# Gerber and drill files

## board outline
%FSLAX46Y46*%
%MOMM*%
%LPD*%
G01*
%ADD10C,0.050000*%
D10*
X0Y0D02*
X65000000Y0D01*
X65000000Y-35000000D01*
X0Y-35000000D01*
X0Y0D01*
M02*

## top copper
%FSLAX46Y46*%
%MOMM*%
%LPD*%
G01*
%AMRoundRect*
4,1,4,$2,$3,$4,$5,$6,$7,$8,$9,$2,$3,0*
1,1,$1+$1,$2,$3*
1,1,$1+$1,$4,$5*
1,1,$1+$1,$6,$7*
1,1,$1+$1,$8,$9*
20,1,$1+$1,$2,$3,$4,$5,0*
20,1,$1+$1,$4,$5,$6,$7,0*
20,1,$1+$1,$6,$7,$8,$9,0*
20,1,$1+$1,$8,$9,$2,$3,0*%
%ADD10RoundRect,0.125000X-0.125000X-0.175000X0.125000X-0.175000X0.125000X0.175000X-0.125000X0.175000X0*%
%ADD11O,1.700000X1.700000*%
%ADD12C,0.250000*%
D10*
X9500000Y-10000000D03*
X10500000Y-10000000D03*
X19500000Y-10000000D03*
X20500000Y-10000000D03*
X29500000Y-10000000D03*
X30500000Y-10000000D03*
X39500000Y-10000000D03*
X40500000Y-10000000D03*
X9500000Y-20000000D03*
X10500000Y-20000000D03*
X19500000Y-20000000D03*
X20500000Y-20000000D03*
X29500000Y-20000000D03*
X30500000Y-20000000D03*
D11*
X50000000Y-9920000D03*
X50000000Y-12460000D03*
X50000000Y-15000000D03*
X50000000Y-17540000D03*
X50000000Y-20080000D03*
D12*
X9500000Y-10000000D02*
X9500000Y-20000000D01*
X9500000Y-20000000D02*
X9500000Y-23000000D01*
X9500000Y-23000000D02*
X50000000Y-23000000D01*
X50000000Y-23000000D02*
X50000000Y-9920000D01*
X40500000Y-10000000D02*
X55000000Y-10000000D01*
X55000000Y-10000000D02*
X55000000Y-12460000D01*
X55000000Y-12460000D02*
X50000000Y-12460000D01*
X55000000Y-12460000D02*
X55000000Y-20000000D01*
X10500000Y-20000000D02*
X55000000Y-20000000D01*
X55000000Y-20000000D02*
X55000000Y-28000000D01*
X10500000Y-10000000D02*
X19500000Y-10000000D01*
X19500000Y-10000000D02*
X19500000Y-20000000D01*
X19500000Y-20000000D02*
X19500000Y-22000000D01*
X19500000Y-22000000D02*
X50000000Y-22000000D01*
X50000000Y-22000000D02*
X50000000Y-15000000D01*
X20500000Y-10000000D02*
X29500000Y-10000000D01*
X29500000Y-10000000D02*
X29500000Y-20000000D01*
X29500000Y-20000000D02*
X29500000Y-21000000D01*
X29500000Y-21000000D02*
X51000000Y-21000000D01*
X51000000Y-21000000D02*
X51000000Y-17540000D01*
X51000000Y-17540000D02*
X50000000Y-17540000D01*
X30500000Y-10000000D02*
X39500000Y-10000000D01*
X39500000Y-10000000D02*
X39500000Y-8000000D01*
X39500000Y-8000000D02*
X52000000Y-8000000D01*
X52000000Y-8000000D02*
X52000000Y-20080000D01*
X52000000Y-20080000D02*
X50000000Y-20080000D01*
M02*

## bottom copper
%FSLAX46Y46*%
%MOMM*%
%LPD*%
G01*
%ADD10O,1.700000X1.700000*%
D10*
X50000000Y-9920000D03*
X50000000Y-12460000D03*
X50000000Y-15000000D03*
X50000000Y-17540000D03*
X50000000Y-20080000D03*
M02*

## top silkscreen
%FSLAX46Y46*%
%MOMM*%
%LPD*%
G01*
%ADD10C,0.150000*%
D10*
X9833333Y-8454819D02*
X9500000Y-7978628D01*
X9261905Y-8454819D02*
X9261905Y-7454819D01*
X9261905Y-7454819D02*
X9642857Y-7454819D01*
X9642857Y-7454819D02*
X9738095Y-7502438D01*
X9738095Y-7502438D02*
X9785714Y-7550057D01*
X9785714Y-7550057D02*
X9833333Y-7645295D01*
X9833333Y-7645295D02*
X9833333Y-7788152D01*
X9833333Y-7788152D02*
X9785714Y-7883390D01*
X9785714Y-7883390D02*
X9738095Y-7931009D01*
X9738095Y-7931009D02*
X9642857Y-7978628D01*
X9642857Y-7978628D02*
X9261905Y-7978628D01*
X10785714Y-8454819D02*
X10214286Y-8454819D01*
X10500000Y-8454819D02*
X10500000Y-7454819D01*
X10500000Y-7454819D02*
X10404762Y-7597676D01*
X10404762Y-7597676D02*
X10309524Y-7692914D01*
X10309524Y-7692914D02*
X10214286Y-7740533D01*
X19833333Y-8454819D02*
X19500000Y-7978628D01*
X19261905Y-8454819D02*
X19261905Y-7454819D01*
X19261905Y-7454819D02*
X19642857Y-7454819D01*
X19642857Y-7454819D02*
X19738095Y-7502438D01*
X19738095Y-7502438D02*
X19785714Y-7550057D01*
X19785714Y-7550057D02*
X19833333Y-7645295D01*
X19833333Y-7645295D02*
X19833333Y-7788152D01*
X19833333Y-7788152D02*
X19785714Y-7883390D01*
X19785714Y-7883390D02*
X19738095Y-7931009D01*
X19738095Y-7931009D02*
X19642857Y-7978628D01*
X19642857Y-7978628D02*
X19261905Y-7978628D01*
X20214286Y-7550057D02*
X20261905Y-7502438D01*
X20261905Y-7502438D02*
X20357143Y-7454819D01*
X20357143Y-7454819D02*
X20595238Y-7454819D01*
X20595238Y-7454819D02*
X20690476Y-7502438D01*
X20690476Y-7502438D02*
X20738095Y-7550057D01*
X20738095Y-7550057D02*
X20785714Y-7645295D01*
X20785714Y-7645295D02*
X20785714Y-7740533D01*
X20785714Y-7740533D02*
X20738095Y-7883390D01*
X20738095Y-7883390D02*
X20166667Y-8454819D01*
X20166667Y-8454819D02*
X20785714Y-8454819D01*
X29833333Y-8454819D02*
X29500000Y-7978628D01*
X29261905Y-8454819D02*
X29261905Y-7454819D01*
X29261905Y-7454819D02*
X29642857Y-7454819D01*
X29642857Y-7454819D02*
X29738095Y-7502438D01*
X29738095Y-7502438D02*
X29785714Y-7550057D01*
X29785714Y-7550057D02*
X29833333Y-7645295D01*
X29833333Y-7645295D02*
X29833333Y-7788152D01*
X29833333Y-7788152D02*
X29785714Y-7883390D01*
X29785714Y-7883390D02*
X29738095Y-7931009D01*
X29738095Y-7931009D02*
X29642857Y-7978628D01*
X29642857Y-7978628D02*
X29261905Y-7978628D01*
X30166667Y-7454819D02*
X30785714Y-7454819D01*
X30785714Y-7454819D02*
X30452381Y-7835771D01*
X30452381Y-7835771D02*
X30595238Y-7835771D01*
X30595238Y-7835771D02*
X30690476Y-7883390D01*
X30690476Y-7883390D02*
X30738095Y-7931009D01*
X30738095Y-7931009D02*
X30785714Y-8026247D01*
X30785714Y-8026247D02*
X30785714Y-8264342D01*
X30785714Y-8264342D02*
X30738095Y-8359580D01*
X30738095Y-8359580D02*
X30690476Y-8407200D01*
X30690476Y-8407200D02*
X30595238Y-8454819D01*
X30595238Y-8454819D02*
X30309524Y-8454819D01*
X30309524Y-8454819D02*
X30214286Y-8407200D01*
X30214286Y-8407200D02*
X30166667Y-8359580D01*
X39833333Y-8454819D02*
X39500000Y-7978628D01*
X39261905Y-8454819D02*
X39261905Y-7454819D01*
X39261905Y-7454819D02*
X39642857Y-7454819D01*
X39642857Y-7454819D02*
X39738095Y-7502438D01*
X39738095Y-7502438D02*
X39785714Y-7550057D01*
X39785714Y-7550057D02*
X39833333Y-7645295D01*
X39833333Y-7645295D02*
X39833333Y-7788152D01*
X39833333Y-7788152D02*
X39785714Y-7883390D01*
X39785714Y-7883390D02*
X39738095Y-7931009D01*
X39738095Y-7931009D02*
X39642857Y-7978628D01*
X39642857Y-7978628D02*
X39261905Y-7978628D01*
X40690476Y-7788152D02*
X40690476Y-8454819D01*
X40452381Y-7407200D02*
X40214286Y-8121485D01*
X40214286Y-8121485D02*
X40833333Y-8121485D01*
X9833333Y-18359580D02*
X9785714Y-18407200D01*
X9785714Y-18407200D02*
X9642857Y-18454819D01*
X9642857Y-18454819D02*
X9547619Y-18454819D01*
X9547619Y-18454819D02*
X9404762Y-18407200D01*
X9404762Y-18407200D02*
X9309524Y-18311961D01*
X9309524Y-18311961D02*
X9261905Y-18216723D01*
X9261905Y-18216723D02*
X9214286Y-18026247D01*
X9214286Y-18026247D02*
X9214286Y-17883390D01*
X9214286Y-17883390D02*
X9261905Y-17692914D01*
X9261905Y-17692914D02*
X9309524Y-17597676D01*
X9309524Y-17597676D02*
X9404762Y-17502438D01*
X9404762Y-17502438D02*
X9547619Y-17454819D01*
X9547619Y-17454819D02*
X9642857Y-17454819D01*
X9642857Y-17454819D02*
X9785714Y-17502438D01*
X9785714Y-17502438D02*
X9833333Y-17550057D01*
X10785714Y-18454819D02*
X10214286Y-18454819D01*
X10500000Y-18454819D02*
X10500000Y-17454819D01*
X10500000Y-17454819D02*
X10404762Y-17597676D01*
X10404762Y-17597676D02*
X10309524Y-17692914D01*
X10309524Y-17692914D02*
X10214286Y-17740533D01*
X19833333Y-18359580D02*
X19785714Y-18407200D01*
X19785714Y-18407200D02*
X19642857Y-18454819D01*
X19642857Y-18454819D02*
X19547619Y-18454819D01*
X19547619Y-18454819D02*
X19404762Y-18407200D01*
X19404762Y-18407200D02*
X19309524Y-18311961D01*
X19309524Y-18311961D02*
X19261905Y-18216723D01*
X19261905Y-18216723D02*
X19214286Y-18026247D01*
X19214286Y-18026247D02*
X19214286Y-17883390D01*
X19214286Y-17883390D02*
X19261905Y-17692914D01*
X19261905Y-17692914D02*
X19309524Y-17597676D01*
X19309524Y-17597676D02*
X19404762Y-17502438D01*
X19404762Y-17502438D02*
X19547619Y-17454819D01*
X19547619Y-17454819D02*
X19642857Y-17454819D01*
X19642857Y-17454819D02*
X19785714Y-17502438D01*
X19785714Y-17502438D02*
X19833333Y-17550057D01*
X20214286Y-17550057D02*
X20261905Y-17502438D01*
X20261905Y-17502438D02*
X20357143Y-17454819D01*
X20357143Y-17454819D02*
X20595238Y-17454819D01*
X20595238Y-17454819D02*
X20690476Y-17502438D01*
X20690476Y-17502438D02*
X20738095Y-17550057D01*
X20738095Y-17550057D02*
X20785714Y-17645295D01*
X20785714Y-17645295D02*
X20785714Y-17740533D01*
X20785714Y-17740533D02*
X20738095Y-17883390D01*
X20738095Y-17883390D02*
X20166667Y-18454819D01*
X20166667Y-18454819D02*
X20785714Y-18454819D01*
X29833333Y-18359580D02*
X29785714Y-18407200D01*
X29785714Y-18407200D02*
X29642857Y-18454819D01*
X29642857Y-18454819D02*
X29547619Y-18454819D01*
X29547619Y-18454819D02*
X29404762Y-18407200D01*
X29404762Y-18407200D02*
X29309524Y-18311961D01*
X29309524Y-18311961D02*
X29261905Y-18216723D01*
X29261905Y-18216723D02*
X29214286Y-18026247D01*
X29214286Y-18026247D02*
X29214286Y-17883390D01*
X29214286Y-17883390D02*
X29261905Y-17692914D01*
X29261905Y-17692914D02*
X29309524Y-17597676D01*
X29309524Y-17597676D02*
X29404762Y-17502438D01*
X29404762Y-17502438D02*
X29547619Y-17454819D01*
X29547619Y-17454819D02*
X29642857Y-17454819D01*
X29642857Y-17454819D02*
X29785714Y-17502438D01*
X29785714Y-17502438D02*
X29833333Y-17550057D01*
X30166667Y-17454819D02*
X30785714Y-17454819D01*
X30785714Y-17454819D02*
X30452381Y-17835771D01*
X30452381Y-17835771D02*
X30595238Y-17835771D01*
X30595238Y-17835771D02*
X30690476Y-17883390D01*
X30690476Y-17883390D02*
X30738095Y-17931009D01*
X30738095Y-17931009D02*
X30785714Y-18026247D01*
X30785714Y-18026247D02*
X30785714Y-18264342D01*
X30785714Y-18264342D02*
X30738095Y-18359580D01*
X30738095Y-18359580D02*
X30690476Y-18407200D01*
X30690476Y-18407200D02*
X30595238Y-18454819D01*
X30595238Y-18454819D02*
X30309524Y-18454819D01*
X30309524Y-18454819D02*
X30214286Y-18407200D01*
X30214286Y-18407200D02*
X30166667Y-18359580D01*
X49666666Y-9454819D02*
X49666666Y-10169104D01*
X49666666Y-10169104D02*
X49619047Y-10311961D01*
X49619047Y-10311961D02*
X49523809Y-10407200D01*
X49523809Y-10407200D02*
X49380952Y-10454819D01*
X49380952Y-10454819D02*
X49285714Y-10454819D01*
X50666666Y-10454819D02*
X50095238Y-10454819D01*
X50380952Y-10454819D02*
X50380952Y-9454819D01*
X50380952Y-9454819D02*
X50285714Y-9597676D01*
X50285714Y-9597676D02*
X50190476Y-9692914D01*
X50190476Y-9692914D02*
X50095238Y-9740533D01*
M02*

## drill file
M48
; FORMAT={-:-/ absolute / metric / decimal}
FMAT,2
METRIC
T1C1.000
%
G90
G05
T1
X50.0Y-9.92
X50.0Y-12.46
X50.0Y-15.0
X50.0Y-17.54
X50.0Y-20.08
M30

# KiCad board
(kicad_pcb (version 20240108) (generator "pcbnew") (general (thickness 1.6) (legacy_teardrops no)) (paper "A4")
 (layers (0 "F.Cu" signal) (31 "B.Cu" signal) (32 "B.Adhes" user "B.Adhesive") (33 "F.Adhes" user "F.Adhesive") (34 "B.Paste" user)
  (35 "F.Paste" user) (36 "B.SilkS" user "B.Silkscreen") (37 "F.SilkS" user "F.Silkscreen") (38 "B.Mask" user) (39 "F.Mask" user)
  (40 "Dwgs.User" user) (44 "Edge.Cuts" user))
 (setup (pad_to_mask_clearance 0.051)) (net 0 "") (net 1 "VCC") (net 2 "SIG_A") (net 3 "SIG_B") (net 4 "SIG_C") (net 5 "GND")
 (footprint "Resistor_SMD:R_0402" (layer "F.Cu") (at 10 10)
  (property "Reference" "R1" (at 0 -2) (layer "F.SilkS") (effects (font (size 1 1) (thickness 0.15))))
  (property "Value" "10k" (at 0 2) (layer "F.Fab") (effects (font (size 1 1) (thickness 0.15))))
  (pad "1" smd roundrect (at -0.5 0) (size 0.5 0.6) (layers "F.Cu" "F.Paste" "F.Mask") (roundrect_rratio 0.25) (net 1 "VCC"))
  (pad "2" smd roundrect (at 0.5 0) (size 0.5 0.6) (layers "F.Cu" "F.Paste" "F.Mask") (roundrect_rratio 0.25) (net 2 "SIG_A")))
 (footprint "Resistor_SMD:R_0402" (layer "F.Cu") (at 20 10)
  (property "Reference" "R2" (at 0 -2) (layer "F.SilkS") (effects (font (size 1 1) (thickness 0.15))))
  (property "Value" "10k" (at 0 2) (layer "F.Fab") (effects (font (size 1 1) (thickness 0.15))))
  (pad "1" smd roundrect (at -0.5 0) (size 0.5 0.6) (layers "F.Cu" "F.Paste" "F.Mask") (roundrect_rratio 0.25) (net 2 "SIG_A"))
  (pad "2" smd roundrect (at 0.5 0) (size 0.5 0.6) (layers "F.Cu" "F.Paste" "F.Mask") (roundrect_rratio 0.25) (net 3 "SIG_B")))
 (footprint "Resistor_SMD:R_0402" (layer "F.Cu") (at 30 10)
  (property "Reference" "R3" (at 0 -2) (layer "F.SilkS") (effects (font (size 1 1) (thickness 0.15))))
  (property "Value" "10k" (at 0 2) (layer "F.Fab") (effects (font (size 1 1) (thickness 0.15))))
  (pad "1" smd roundrect (at -0.5 0) (size 0.5 0.6) (layers "F.Cu" "F.Paste" "F.Mask") (roundrect_rratio 0.25) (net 3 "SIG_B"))
  (pad "2" smd roundrect (at 0.5 0) (size 0.5 0.6) (layers "F.Cu" "F.Paste" "F.Mask") (roundrect_rratio 0.25) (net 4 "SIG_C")))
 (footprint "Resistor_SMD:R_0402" (layer "F.Cu") (at 40 10)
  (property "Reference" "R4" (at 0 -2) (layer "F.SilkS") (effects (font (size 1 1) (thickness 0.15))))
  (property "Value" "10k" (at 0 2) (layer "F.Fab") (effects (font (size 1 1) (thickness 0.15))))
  (pad "1" smd roundrect (at -0.5 0) (size 0.5 0.6) (layers "F.Cu" "F.Paste" "F.Mask") (roundrect_rratio 0.25) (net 4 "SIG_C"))
  (pad "2" smd roundrect (at 0.5 0) (size 0.5 0.6) (layers "F.Cu" "F.Paste" "F.Mask") (roundrect_rratio 0.25) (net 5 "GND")))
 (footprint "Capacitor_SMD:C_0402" (layer "F.Cu") (at 10 20)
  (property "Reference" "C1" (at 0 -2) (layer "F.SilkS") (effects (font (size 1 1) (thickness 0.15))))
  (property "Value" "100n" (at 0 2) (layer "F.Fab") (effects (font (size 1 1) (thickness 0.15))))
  (pad "1" smd roundrect (at -0.5 0) (size 0.5 0.6) (layers "F.Cu" "F.Paste" "F.Mask") (roundrect_rratio 0.25) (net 1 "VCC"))
  (pad "2" smd roundrect (at 0.5 0) (size 0.5 0.6) (layers "F.Cu" "F.Paste" "F.Mask") (roundrect_rratio 0.25) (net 5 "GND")))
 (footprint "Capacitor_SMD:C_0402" (layer "F.Cu") (at 20 20)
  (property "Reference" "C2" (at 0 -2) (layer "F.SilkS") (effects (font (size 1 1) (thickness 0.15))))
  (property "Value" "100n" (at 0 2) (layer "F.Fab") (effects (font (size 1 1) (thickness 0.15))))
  (pad "1" smd roundrect (at -0.5 0) (size 0.5 0.6) (layers "F.Cu" "F.Paste" "F.Mask") (roundrect_rratio 0.25) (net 2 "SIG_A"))
  (pad "2" smd roundrect (at 0.5 0) (size 0.5 0.6) (layers "F.Cu" "F.Paste" "F.Mask") (roundrect_rratio 0.25) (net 5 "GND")))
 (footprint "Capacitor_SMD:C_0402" (layer "F.Cu") (at 30 20)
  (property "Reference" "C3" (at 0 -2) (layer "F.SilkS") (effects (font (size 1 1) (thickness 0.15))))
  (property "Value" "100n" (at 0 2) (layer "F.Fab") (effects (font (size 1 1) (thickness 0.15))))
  (pad "1" smd roundrect (at -0.5 0) (size 0.5 0.6) (layers "F.Cu" "F.Paste" "F.Mask") (roundrect_rratio 0.25) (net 3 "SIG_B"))
  (pad "2" smd roundrect (at 0.5 0) (size 0.5 0.6) (layers "F.Cu" "F.Paste" "F.Mask") (roundrect_rratio 0.25) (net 5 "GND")))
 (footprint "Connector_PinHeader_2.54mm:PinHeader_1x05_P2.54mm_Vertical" (layer "F.Cu") (at 50 15)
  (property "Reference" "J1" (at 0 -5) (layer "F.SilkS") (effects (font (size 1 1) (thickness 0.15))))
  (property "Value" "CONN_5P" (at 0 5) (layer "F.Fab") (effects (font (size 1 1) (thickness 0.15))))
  (pad "1" thru_hole oval (at 0 -5.08) (size 1.7 1.7) (drill 1.0) (layers "*.Cu" "*.Mask") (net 1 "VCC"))
  (pad "2" thru_hole oval (at 0 -2.54) (size 1.7 1.7) (drill 1.0) (layers "*.Cu" "*.Mask") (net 5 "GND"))
  (pad "3" thru_hole oval (at 0 0) (size 1.7 1.7) (drill 1.0) (layers "*.Cu" "*.Mask") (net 2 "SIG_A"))
  (pad "4" thru_hole oval (at 0 2.54) (size 1.7 1.7) (drill 1.0) (layers "*.Cu" "*.Mask") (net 3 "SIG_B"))
  (pad "5" thru_hole oval (at 0 5.08) (size 1.7 1.7) (drill 1.0) (layers "*.Cu" "*.Mask") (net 4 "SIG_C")))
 (gr_rect (start 0 0) (end 65 35) (layer "Edge.Cuts") (width 0.05))
 (segment (start 9.5 10) (end 9.5 20) (width 0.25) (layer "F.Cu") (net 1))
 (segment (start 9.5 20) (end 9.5 23) (width 0.25) (layer "F.Cu") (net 1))
 (segment (start 9.5 23) (end 50 23) (width 0.25) (layer "F.Cu") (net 1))
 (segment (start 50 23) (end 50 9.92) (width 0.25) (layer "F.Cu") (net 1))
 (segment (start 40.5 10) (end 55 10) (width 0.25) (layer "F.Cu") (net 5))
 (segment (start 55 10) (end 55 12.46) (width 0.25) (layer "F.Cu") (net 5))
 (segment (start 55 12.46) (end 50 12.46) (width 0.25) (layer "F.Cu") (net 5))
 (segment (start 55 12.46) (end 55 20) (width 0.25) (layer "F.Cu") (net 5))
 (segment (start 10.5 20) (end 55 20) (width 0.25) (layer "F.Cu") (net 5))
 (segment (start 55 20) (end 55 28) (width 0.25) (layer "F.Cu") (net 5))
 (segment (start 10.5 10) (end 19.5 10) (width 0.25) (layer "F.Cu") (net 2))
 (segment (start 19.5 10) (end 19.5 20) (width 0.25) (layer "F.Cu") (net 2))
 (segment (start 19.5 20) (end 19.5 22) (width 0.25) (layer "F.Cu") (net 2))
 (segment (start 19.5 22) (end 50 22) (width 0.25) (layer "F.Cu") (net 2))
 (segment (start 50 22) (end 50 15) (width 0.25) (layer "F.Cu") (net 2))
 (segment (start 20.5 10) (end 29.5 10) (width 0.25) (layer "F.Cu") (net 3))
 (segment (start 29.5 10) (end 29.5 20) (width 0.25) (layer "F.Cu") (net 3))
 (segment (start 29.5 20) (end 29.5 21) (width 0.25) (layer "F.Cu") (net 3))
 (segment (start 29.5 21) (end 51 21) (width 0.25) (layer "F.Cu") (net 3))
 (segment (start 51 21) (end 51 17.54) (width 0.25) (layer "F.Cu") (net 3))
 (segment (start 51 17.54) (end 50 17.54) (width 0.25) (layer "F.Cu") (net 3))
 (segment (start 30.5 10) (end 39.5 10) (width 0.25) (layer "F.Cu") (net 4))
 (segment (start 39.5 10) (end 39.5 8) (width 0.25) (layer "F.Cu") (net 4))
 (segment (start 39.5 8) (end 52 8) (width 0.25) (layer "F.Cu") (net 4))
 (segment (start 52 8) (end 52 20.08) (width 0.25) (layer "F.Cu") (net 4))
 (segment (start 52 20.08) (end 50 20.08) (width 0.25) (layer "F.Cu") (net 4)))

